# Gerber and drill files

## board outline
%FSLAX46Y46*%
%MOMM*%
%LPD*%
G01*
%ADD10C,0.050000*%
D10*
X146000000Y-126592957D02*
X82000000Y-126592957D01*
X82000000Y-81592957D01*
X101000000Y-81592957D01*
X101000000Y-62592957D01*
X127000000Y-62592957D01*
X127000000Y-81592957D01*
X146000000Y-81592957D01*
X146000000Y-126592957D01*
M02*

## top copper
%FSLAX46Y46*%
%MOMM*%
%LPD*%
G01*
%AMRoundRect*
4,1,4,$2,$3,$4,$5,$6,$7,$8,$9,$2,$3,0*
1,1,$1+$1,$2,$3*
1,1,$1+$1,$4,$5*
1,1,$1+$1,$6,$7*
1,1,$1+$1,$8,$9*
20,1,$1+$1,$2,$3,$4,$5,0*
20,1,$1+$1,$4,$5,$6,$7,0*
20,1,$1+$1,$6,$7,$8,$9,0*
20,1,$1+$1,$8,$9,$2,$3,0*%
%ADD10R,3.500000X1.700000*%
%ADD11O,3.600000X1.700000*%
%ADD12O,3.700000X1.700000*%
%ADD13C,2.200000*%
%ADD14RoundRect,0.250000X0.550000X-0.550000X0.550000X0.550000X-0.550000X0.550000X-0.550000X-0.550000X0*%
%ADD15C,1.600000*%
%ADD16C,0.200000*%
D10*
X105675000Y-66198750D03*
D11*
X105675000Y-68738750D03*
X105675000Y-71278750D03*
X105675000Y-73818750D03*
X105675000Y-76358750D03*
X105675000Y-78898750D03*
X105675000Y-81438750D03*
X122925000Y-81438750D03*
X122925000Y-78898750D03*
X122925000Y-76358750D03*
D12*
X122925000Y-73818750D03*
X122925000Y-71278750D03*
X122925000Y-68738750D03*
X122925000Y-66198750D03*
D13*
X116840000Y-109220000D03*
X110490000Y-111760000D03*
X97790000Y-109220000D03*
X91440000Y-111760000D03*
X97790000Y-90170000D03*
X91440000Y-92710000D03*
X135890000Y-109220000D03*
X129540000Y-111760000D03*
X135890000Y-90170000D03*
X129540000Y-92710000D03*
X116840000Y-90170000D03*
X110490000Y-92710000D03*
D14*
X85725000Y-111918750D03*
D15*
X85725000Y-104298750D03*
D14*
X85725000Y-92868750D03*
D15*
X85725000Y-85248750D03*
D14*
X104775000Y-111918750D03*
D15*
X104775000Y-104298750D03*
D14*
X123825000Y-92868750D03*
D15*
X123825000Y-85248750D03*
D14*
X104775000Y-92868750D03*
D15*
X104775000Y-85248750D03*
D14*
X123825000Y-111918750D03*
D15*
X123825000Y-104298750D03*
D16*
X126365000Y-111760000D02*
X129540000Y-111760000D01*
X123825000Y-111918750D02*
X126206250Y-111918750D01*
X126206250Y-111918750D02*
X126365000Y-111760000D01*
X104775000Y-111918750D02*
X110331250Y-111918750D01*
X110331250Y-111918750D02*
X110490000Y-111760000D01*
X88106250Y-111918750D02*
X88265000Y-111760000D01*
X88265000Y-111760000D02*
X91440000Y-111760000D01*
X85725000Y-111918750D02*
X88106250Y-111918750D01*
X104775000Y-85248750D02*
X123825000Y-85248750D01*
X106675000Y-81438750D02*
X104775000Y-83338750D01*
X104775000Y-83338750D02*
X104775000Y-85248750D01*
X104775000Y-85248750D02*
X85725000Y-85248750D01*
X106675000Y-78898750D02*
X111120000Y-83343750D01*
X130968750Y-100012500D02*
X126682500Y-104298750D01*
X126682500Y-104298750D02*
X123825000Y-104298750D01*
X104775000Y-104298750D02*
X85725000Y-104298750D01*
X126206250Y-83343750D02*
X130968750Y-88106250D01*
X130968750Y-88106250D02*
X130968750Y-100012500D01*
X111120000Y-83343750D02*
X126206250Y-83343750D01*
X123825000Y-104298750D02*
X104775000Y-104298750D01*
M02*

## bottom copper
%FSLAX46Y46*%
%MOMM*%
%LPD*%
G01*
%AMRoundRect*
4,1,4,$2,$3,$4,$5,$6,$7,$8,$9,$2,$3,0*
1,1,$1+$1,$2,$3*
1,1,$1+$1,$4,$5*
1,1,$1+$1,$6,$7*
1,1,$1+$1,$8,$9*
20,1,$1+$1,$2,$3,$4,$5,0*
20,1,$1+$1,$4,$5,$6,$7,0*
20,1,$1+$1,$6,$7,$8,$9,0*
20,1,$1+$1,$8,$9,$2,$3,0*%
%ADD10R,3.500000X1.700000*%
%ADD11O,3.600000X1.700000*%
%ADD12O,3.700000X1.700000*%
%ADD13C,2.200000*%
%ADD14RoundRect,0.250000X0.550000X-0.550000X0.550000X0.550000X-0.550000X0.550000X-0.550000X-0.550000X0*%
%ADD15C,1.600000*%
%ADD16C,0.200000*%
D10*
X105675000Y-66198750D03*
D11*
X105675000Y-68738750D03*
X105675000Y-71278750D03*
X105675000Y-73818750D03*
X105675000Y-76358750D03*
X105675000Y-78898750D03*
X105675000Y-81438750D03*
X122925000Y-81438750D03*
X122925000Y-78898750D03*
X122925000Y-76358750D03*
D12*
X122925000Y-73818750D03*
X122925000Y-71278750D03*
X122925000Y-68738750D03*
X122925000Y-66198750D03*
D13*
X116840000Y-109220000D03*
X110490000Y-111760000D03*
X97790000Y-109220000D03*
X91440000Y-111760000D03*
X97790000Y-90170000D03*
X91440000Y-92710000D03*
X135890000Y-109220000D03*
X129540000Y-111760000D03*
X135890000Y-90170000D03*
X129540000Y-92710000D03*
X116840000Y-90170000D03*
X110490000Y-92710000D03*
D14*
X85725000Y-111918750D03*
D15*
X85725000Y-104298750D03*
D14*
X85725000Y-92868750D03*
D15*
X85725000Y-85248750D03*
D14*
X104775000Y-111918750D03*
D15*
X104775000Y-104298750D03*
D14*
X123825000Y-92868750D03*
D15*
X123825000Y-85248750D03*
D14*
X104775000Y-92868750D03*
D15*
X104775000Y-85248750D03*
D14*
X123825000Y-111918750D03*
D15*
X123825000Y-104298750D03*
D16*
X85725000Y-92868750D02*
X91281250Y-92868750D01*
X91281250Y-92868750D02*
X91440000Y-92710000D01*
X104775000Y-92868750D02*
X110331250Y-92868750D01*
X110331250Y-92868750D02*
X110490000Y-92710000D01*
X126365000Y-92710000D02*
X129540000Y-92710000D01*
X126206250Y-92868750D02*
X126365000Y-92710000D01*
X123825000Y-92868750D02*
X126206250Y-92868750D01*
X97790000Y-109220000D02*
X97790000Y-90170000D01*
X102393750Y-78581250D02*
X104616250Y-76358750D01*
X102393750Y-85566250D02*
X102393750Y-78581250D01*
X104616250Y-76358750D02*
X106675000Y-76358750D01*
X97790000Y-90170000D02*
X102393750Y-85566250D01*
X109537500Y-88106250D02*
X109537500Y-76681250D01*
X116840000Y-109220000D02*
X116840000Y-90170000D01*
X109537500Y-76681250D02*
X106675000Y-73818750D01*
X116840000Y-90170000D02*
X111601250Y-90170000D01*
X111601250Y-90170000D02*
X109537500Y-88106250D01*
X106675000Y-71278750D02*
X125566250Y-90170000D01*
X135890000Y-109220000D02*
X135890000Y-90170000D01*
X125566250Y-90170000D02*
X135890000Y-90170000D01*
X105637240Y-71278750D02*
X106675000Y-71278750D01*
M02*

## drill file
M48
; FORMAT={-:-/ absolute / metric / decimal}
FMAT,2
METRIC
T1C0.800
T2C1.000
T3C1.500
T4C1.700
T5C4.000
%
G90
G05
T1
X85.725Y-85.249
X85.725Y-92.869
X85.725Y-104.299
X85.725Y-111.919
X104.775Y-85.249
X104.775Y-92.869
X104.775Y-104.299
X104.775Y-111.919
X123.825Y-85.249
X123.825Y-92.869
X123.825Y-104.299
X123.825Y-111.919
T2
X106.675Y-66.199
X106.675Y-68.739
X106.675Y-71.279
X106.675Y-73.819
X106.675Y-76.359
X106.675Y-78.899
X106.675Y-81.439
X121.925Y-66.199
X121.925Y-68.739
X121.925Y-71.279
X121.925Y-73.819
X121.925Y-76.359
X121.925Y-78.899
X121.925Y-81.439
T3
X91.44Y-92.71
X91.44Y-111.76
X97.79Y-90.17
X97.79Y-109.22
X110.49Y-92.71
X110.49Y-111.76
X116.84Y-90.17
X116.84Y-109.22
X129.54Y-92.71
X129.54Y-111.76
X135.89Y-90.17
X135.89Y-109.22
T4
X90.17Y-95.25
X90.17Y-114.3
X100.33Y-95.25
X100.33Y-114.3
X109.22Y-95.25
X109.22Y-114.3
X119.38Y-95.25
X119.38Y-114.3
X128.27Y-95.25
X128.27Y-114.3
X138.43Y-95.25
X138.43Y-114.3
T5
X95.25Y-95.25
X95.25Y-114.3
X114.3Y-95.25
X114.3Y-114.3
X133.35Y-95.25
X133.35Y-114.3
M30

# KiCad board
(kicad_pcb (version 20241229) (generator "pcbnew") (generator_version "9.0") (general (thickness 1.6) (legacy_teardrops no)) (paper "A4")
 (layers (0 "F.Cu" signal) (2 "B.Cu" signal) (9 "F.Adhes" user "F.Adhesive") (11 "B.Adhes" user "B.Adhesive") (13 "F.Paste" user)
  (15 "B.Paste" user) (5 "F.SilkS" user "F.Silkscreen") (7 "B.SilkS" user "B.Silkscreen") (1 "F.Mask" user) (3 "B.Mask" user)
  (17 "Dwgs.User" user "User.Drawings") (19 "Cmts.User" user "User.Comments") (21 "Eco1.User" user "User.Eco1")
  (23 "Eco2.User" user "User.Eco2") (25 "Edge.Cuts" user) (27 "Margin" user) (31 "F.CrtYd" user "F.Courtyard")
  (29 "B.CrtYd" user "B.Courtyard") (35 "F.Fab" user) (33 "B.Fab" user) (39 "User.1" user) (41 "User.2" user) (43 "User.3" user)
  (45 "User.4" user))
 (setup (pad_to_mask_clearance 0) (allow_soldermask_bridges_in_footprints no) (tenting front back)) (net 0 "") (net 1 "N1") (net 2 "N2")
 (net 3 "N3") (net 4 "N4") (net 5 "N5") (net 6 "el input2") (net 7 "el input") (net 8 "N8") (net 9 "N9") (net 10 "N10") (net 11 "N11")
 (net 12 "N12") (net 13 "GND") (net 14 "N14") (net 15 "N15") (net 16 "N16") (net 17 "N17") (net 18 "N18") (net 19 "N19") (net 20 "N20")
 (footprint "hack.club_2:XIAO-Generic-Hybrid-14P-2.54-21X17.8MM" (layer "F.Cu") (at 114.3 73.81875)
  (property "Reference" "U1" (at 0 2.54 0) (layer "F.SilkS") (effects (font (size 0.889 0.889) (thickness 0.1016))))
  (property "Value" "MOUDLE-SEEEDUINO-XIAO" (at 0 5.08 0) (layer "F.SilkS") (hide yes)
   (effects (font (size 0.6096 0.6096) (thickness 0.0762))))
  (pad "1" thru_hole rect (at -7.625 -7.62) (size 3.5 1.7) (drill 1 (offset -1 0)) (layers "*.Cu" "*.Mask") (remove_unused_layers no)
   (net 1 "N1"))
  (pad "2" thru_hole oval (at -7.625 -5.08) (size 3.6 1.7) (drill 1 (offset -1 0)) (layers "*.Cu" "*.Mask") (remove_unused_layers no)
   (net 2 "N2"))
  (pad "3" thru_hole oval (at -7.625 -2.54) (size 3.6 1.7) (drill 1 (offset -1 0)) (layers "*.Cu" "*.Mask") (remove_unused_layers no)
   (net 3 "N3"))
  (pad "4" thru_hole oval (at -7.625 0) (size 3.6 1.7) (drill 1 (offset -1 0)) (layers "*.Cu" "*.Mask") (remove_unused_layers no)
   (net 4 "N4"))
  (pad "5" thru_hole oval (at -7.625 2.54) (size 3.6 1.7) (drill 1 (offset -1 0)) (layers "*.Cu" "*.Mask") (remove_unused_layers no)
   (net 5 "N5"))
  (pad "6" thru_hole oval (at -7.625 5.08 180) (size 3.6 1.7) (drill 1 (offset 1 0)) (layers "*.Cu" "*.Mask") (remove_unused_layers no)
   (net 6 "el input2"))
  (pad "7" thru_hole oval (at -7.625 7.62) (size 3.6 1.7) (drill 1 (offset -1 0)) (layers "*.Cu" "*.Mask") (remove_unused_layers no)
   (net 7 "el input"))
  (pad "8" thru_hole oval (at 7.625 7.62) (size 3.6 1.7) (drill 1 (offset 1 0)) (layers "*.Cu" "*.Mask") (remove_unused_layers no)
   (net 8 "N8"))
  (pad "9" thru_hole oval (at 7.625 5.08) (size 3.6 1.7) (drill 1 (offset 1 0)) (layers "*.Cu" "*.Mask") (remove_unused_layers no)
   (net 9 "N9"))
  (pad "10" thru_hole oval (at 7.625 2.54) (size 3.6 1.7) (drill 1 (offset 1 0)) (layers "*.Cu" "*.Mask") (remove_unused_layers no)
   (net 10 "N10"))
  (pad "11" thru_hole oval (at 7.625 0) (size 3.7 1.7) (drill 1 (offset 1 0)) (layers "*.Cu" "*.Mask") (remove_unused_layers no)
   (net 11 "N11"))
  (pad "12" thru_hole oval (at 7.625 -2.54) (size 3.7 1.7) (drill 1 (offset 1 0)) (layers "*.Cu" "*.Mask") (remove_unused_layers no)
   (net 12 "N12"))
  (pad "13" thru_hole oval (at 7.625 -5.08) (size 3.7 1.7) (drill 1 (offset 1 0)) (layers "*.Cu" "*.Mask") (remove_unused_layers no)
   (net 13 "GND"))
  (pad "14" thru_hole oval (at 7.625 -7.62) (size 3.7 1.7) (drill 1 (offset 1 0)) (layers "*.Cu" "*.Mask") (remove_unused_layers no)
   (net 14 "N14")))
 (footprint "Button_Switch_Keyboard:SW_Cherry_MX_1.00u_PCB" (layer "F.Cu") (at 116.84 109.22)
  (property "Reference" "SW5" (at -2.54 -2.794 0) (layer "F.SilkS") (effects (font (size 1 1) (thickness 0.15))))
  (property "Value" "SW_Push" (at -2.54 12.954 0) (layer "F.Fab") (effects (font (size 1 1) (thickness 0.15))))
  (pad "" np_thru_hole circle (at -7.62 5.08) (size 1.7 1.7) (drill 1.7) (layers "*.Cu" "*.Mask"))
  (pad "" np_thru_hole circle (at -2.54 5.08) (size 4 4) (drill 4) (layers "*.Cu" "*.Mask"))
  (pad "" np_thru_hole circle (at 2.54 5.08) (size 1.7 1.7) (drill 1.7) (layers "*.Cu" "*.Mask"))
  (pad "1" thru_hole circle (at 0 0) (size 2.2 2.2) (drill 1.5) (layers "*.Cu" "*.Mask") (remove_unused_layers no) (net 4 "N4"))
  (pad "2" thru_hole circle (at -6.35 2.54) (size 2.2 2.2) (drill 1.5) (layers "*.Cu" "*.Mask") (remove_unused_layers no) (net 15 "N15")))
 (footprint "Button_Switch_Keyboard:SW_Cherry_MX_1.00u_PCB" (layer "F.Cu") (at 97.79 109.22)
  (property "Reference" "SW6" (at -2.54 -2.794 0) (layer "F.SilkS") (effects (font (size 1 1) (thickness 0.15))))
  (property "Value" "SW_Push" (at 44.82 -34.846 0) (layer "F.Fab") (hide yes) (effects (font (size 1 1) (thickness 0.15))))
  (pad "" np_thru_hole circle (at -7.62 5.08) (size 1.7 1.7) (drill 1.7) (layers "*.Cu" "*.Mask"))
  (pad "" np_thru_hole circle (at -2.54 5.08) (size 4 4) (drill 4) (layers "*.Cu" "*.Mask"))
  (pad "" np_thru_hole circle (at 2.54 5.08) (size 1.7 1.7) (drill 1.7) (layers "*.Cu" "*.Mask"))
  (pad "1" thru_hole circle (at 0 0) (size 2.2 2.2) (drill 1.5) (layers "*.Cu" "*.Mask") (remove_unused_layers no) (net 5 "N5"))
  (pad "2" thru_hole circle (at -6.35 2.54) (size 2.2 2.2) (drill 1.5) (layers "*.Cu" "*.Mask") (remove_unused_layers no) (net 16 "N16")))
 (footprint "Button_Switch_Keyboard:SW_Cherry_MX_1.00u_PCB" (layer "F.Cu") (at 97.79 90.17)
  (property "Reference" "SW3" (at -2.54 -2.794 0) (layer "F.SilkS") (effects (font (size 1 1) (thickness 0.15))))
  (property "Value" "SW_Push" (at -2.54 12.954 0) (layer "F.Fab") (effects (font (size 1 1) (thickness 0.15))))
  (pad "" np_thru_hole circle (at -7.62 5.08) (size 1.7 1.7) (drill 1.7) (layers "*.Cu" "*.Mask"))
  (pad "" np_thru_hole circle (at -2.54 5.08) (size 4 4) (drill 4) (layers "*.Cu" "*.Mask"))
  (pad "" np_thru_hole circle (at 2.54 5.08) (size 1.7 1.7) (drill 1.7) (layers "*.Cu" "*.Mask"))
  (pad "1" thru_hole circle (at 0 0) (size 2.2 2.2) (drill 1.5) (layers "*.Cu" "*.Mask") (remove_unused_layers no) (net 5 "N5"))
  (pad "2" thru_hole circle (at -6.35 2.54) (size 2.2 2.2) (drill 1.5) (layers "*.Cu" "*.Mask") (remove_unused_layers no) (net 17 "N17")))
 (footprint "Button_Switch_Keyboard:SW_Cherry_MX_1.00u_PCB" (layer "F.Cu") (at 135.89 109.22)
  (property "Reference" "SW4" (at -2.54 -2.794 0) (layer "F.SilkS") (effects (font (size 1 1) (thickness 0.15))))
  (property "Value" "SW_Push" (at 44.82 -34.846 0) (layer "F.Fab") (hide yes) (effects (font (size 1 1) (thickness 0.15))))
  (pad "" np_thru_hole circle (at -7.62 5.08) (size 1.7 1.7) (drill 1.7) (layers "*.Cu" "*.Mask"))
  (pad "" np_thru_hole circle (at -2.54 5.08) (size 4 4) (drill 4) (layers "*.Cu" "*.Mask"))
  (pad "" np_thru_hole circle (at 2.54 5.08) (size 1.7 1.7) (drill 1.7) (layers "*.Cu" "*.Mask"))
  (pad "1" thru_hole circle (at 0 0) (size 2.2 2.2) (drill 1.5) (layers "*.Cu" "*.Mask") (remove_unused_layers no) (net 3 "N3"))
  (pad "2" thru_hole circle (at -6.35 2.54) (size 2.2 2.2) (drill 1.5) (layers "*.Cu" "*.Mask") (remove_unused_layers no) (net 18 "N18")))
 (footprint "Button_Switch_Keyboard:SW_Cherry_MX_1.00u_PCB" (layer "F.Cu") (at 135.89 90.17)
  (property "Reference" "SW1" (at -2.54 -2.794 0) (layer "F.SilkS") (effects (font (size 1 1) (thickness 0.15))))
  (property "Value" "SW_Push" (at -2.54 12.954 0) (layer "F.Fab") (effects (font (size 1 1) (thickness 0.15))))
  (pad "" np_thru_hole circle (at -7.62 5.08) (size 1.7 1.7) (drill 1.7) (layers "*.Cu" "*.Mask"))
  (pad "" np_thru_hole circle (at -2.54 5.08) (size 4 4) (drill 4) (layers "*.Cu" "*.Mask"))
  (pad "" np_thru_hole circle (at 2.54 5.08) (size 1.7 1.7) (drill 1.7) (layers "*.Cu" "*.Mask"))
  (pad "1" thru_hole circle (at 0 0) (size 2.2 2.2) (drill 1.5) (layers "*.Cu" "*.Mask") (remove_unused_layers no) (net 3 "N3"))
  (pad "2" thru_hole circle (at -6.35 2.54) (size 2.2 2.2) (drill 1.5) (layers "*.Cu" "*.Mask") (remove_unused_layers no) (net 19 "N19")))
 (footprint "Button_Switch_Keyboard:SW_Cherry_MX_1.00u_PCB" (layer "F.Cu") (at 116.84 90.17)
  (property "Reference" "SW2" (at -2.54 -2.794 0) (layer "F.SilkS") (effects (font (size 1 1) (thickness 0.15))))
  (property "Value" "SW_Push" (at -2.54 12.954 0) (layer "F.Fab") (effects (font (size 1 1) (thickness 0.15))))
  (pad "" np_thru_hole circle (at -7.62 5.08) (size 1.7 1.7) (drill 1.7) (layers "*.Cu" "*.Mask"))
  (pad "" np_thru_hole circle (at -2.54 5.08) (size 4 4) (drill 4) (layers "*.Cu" "*.Mask"))
  (pad "" np_thru_hole circle (at 2.54 5.08) (size 1.7 1.7) (drill 1.7) (layers "*.Cu" "*.Mask"))
  (pad "1" thru_hole circle (at 0 0) (size 2.2 2.2) (drill 1.5) (layers "*.Cu" "*.Mask") (remove_unused_layers no) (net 4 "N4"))
  (pad "2" thru_hole circle (at -6.35 2.54) (size 2.2 2.2) (drill 1.5) (layers "*.Cu" "*.Mask") (remove_unused_layers no) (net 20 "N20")))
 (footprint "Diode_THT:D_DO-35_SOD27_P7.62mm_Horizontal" (layer "B.Cu") (at 85.725 111.91875 90)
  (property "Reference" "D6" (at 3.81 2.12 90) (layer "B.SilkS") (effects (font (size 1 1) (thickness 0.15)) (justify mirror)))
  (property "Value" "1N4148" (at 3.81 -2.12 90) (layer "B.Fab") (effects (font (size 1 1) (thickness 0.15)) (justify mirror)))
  (pad "1" thru_hole roundrect (at 0 0 90) (size 1.6 1.6) (drill 0.8) (layers "*.Cu" "*.Mask") (remove_unused_layers no)
   (roundrect_rratio 0.15625) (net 16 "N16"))
  (pad "2" thru_hole circle (at 7.62 0 90) (size 1.6 1.6) (drill 0.8) (layers "*.Cu" "*.Mask") (remove_unused_layers no) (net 6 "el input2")))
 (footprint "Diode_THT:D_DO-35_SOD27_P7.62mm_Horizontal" (layer "B.Cu") (at 85.725 92.86875 90)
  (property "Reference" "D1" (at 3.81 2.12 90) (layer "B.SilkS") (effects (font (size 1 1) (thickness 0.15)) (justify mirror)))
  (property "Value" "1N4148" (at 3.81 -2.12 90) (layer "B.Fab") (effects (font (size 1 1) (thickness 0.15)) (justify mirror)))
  (pad "1" thru_hole roundrect (at 0 0 90) (size 1.6 1.6) (drill 0.8) (layers "*.Cu" "*.Mask") (remove_unused_layers no)
   (roundrect_rratio 0.15625) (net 17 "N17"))
  (pad "2" thru_hole circle (at 7.62 0 90) (size 1.6 1.6) (drill 0.8) (layers "*.Cu" "*.Mask") (remove_unused_layers no) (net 7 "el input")))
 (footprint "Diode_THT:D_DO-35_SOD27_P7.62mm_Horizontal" (layer "B.Cu") (at 104.775 111.91875 90)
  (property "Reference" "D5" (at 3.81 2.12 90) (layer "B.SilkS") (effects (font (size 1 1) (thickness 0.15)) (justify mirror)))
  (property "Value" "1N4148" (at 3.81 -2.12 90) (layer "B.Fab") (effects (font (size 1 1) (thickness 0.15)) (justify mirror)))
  (pad "1" thru_hole roundrect (at 0 0 90) (size 1.6 1.6) (drill 0.8) (layers "*.Cu" "*.Mask") (remove_unused_layers no)
   (roundrect_rratio 0.15625) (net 15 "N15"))
  (pad "2" thru_hole circle (at 7.62 0 90) (size 1.6 1.6) (drill 0.8) (layers "*.Cu" "*.Mask") (remove_unused_layers no) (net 6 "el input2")))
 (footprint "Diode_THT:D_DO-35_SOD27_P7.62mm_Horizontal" (layer "B.Cu") (at 123.825 92.86875 90)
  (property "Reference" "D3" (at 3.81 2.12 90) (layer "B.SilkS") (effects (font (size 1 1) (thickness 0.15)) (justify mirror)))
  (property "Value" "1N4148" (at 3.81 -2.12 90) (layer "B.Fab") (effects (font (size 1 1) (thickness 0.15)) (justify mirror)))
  (pad "1" thru_hole roundrect (at 0 0 90) (size 1.6 1.6) (drill 0.8) (layers "*.Cu" "*.Mask") (remove_unused_layers no)
   (roundrect_rratio 0.15625) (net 19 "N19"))
  (pad "2" thru_hole circle (at 7.62 0 90) (size 1.6 1.6) (drill 0.8) (layers "*.Cu" "*.Mask") (remove_unused_layers no) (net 7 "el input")))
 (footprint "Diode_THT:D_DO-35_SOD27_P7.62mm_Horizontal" (layer "B.Cu") (at 104.775 92.86875 90)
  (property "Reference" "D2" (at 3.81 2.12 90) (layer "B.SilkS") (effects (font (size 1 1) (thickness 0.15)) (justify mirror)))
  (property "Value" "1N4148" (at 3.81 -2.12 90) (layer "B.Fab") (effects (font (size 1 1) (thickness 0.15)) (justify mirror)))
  (pad "1" thru_hole roundrect (at 0 0 90) (size 1.6 1.6) (drill 0.8) (layers "*.Cu" "*.Mask") (remove_unused_layers no)
   (roundrect_rratio 0.15625) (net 20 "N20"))
  (pad "2" thru_hole circle (at 7.62 0 90) (size 1.6 1.6) (drill 0.8) (layers "*.Cu" "*.Mask") (remove_unused_layers no) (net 7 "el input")))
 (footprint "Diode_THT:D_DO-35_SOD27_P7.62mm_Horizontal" (layer "B.Cu") (at 123.825 111.91875 90)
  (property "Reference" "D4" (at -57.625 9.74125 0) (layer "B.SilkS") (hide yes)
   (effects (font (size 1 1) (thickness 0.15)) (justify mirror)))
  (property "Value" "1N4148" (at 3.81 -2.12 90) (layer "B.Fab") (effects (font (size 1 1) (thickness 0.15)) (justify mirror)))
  (pad "1" thru_hole roundrect (at 0 0 90) (size 1.6 1.6) (drill 0.8) (layers "*.Cu" "*.Mask") (remove_unused_layers no)
   (roundrect_rratio 0.15625) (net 18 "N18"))
  (pad "2" thru_hole circle (at 7.62 0 90) (size 1.6 1.6) (drill 0.8) (layers "*.Cu" "*.Mask") (remove_unused_layers no) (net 6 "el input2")))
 (gr_poly
  (pts (xy 146 126.592957) (xy 82 126.592957) (xy 82 81.592957) (xy 101 81.592957) (xy 101 62.592957) (xy 127 62.592957) (xy 127 81.592957)
   (xy 146 81.592957))
  (stroke (width 0.05) (type solid)) (fill no) (layer "Edge.Cuts"))
 (segment (start 85.725 92.86875) (end 91.28125 92.86875) (width 0.2) (layer "B.Cu") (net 17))
 (segment (start 91.28125 92.86875) (end 91.44 92.71) (width 0.2) (layer "B.Cu") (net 17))
 (segment (start 104.775 92.86875) (end 110.33125 92.86875) (width 0.2) (layer "B.Cu") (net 20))
 (segment (start 110.33125 92.86875) (end 110.49 92.71) (width 0.2) (layer "B.Cu") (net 20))
 (segment (start 126.365 92.71) (end 129.54 92.71) (width 0.2) (layer "B.Cu") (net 19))
 (segment (start 126.20625 92.86875) (end 126.365 92.71) (width 0.2) (layer "B.Cu") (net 19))
 (segment (start 123.825 92.86875) (end 126.20625 92.86875) (width 0.2) (layer "B.Cu") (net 19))
 (segment (start 126.365 111.76) (end 129.54 111.76) (width 0.2) (layer "F.Cu") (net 18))
 (segment (start 123.825 111.91875) (end 126.20625 111.91875) (width 0.2) (layer "F.Cu") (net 18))
 (segment (start 126.20625 111.91875) (end 126.365 111.76) (width 0.2) (layer "F.Cu") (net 18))
 (segment (start 104.775 111.91875) (end 110.33125 111.91875) (width 0.2) (layer "F.Cu") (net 15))
 (segment (start 110.33125 111.91875) (end 110.49 111.76) (width 0.2) (layer "F.Cu") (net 15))
 (segment (start 88.10625 111.91875) (end 88.265 111.76) (width 0.2) (layer "F.Cu") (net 16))
 (segment (start 88.265 111.76) (end 91.44 111.76) (width 0.2) (layer "F.Cu") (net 16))
 (segment (start 85.725 111.91875) (end 88.10625 111.91875) (width 0.2) (layer "F.Cu") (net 16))
 (segment (start 97.79 109.22) (end 97.79 90.17) (width 0.2) (layer "B.Cu") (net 5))
 (segment (start 102.39375 78.58125) (end 104.61625 76.35875) (width 0.2) (layer "B.Cu") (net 5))
 (segment (start 102.39375 85.56625) (end 102.39375 78.58125) (width 0.2) (layer "B.Cu") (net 5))
 (segment (start 104.61625 76.35875) (end 106.675 76.35875) (width 0.2) (layer "B.Cu") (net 5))
 (segment (start 97.79 90.17) (end 102.39375 85.56625) (width 0.2) (layer "B.Cu") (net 5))
 (segment (start 109.5375 88.10625) (end 109.5375 76.68125) (width 0.2) (layer "B.Cu") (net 4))
 (segment (start 116.84 109.22) (end 116.84 90.17) (width 0.2) (layer "B.Cu") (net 4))
 (segment (start 109.5375 76.68125) (end 106.675 73.81875) (width 0.2) (layer "B.Cu") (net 4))
 (segment (start 116.84 90.17) (end 111.60125 90.17) (width 0.2) (layer "B.Cu") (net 4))
 (segment (start 111.60125 90.17) (end 109.5375 88.10625) (width 0.2) (layer "B.Cu") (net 4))
 (segment (start 106.675 71.27875) (end 125.56625 90.17) (width 0.2) (layer "B.Cu") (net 3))
 (segment (start 135.89 109.22) (end 135.89 90.17) (width 0.2) (layer "B.Cu") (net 3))
 (segment (start 125.56625 90.17) (end 135.89 90.17) (width 0.2) (layer "B.Cu") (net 3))
 (segment (start 105.63724 71.27875) (end 106.675 71.27875) (width 0.2) (layer "B.Cu") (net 3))
 (segment (start 104.775 85.24875) (end 123.825 85.24875) (width 0.2) (layer "F.Cu") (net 7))
 (segment (start 106.675 81.43875) (end 104.775 83.33875) (width 0.2) (layer "F.Cu") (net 7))
 (segment (start 104.775 83.33875) (end 104.775 85.24875) (width 0.2) (layer "F.Cu") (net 7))
 (segment (start 104.775 85.24875) (end 85.725 85.24875) (width 0.2) (layer "F.Cu") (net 7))
 (segment (start 106.675 78.89875) (end 111.12 83.34375) (width 0.2) (layer "F.Cu") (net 6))
 (segment (start 130.96875 100.0125) (end 126.6825 104.29875) (width 0.2) (layer "F.Cu") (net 6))
 (segment (start 126.6825 104.29875) (end 123.825 104.29875) (width 0.2) (layer "F.Cu") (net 6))
 (segment (start 104.775 104.29875) (end 85.725 104.29875) (width 0.2) (layer "F.Cu") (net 6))
 (segment (start 126.20625 83.34375) (end 130.96875 88.10625) (width 0.2) (layer "F.Cu") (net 6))
 (segment (start 130.96875 88.10625) (end 130.96875 100.0125) (width 0.2) (layer "F.Cu") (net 6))
 (segment (start 111.12 83.34375) (end 126.20625 83.34375) (width 0.2) (layer "F.Cu") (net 6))
 (segment (start 123.825 104.29875) (end 104.775 104.29875) (width 0.2) (layer "F.Cu") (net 6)))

